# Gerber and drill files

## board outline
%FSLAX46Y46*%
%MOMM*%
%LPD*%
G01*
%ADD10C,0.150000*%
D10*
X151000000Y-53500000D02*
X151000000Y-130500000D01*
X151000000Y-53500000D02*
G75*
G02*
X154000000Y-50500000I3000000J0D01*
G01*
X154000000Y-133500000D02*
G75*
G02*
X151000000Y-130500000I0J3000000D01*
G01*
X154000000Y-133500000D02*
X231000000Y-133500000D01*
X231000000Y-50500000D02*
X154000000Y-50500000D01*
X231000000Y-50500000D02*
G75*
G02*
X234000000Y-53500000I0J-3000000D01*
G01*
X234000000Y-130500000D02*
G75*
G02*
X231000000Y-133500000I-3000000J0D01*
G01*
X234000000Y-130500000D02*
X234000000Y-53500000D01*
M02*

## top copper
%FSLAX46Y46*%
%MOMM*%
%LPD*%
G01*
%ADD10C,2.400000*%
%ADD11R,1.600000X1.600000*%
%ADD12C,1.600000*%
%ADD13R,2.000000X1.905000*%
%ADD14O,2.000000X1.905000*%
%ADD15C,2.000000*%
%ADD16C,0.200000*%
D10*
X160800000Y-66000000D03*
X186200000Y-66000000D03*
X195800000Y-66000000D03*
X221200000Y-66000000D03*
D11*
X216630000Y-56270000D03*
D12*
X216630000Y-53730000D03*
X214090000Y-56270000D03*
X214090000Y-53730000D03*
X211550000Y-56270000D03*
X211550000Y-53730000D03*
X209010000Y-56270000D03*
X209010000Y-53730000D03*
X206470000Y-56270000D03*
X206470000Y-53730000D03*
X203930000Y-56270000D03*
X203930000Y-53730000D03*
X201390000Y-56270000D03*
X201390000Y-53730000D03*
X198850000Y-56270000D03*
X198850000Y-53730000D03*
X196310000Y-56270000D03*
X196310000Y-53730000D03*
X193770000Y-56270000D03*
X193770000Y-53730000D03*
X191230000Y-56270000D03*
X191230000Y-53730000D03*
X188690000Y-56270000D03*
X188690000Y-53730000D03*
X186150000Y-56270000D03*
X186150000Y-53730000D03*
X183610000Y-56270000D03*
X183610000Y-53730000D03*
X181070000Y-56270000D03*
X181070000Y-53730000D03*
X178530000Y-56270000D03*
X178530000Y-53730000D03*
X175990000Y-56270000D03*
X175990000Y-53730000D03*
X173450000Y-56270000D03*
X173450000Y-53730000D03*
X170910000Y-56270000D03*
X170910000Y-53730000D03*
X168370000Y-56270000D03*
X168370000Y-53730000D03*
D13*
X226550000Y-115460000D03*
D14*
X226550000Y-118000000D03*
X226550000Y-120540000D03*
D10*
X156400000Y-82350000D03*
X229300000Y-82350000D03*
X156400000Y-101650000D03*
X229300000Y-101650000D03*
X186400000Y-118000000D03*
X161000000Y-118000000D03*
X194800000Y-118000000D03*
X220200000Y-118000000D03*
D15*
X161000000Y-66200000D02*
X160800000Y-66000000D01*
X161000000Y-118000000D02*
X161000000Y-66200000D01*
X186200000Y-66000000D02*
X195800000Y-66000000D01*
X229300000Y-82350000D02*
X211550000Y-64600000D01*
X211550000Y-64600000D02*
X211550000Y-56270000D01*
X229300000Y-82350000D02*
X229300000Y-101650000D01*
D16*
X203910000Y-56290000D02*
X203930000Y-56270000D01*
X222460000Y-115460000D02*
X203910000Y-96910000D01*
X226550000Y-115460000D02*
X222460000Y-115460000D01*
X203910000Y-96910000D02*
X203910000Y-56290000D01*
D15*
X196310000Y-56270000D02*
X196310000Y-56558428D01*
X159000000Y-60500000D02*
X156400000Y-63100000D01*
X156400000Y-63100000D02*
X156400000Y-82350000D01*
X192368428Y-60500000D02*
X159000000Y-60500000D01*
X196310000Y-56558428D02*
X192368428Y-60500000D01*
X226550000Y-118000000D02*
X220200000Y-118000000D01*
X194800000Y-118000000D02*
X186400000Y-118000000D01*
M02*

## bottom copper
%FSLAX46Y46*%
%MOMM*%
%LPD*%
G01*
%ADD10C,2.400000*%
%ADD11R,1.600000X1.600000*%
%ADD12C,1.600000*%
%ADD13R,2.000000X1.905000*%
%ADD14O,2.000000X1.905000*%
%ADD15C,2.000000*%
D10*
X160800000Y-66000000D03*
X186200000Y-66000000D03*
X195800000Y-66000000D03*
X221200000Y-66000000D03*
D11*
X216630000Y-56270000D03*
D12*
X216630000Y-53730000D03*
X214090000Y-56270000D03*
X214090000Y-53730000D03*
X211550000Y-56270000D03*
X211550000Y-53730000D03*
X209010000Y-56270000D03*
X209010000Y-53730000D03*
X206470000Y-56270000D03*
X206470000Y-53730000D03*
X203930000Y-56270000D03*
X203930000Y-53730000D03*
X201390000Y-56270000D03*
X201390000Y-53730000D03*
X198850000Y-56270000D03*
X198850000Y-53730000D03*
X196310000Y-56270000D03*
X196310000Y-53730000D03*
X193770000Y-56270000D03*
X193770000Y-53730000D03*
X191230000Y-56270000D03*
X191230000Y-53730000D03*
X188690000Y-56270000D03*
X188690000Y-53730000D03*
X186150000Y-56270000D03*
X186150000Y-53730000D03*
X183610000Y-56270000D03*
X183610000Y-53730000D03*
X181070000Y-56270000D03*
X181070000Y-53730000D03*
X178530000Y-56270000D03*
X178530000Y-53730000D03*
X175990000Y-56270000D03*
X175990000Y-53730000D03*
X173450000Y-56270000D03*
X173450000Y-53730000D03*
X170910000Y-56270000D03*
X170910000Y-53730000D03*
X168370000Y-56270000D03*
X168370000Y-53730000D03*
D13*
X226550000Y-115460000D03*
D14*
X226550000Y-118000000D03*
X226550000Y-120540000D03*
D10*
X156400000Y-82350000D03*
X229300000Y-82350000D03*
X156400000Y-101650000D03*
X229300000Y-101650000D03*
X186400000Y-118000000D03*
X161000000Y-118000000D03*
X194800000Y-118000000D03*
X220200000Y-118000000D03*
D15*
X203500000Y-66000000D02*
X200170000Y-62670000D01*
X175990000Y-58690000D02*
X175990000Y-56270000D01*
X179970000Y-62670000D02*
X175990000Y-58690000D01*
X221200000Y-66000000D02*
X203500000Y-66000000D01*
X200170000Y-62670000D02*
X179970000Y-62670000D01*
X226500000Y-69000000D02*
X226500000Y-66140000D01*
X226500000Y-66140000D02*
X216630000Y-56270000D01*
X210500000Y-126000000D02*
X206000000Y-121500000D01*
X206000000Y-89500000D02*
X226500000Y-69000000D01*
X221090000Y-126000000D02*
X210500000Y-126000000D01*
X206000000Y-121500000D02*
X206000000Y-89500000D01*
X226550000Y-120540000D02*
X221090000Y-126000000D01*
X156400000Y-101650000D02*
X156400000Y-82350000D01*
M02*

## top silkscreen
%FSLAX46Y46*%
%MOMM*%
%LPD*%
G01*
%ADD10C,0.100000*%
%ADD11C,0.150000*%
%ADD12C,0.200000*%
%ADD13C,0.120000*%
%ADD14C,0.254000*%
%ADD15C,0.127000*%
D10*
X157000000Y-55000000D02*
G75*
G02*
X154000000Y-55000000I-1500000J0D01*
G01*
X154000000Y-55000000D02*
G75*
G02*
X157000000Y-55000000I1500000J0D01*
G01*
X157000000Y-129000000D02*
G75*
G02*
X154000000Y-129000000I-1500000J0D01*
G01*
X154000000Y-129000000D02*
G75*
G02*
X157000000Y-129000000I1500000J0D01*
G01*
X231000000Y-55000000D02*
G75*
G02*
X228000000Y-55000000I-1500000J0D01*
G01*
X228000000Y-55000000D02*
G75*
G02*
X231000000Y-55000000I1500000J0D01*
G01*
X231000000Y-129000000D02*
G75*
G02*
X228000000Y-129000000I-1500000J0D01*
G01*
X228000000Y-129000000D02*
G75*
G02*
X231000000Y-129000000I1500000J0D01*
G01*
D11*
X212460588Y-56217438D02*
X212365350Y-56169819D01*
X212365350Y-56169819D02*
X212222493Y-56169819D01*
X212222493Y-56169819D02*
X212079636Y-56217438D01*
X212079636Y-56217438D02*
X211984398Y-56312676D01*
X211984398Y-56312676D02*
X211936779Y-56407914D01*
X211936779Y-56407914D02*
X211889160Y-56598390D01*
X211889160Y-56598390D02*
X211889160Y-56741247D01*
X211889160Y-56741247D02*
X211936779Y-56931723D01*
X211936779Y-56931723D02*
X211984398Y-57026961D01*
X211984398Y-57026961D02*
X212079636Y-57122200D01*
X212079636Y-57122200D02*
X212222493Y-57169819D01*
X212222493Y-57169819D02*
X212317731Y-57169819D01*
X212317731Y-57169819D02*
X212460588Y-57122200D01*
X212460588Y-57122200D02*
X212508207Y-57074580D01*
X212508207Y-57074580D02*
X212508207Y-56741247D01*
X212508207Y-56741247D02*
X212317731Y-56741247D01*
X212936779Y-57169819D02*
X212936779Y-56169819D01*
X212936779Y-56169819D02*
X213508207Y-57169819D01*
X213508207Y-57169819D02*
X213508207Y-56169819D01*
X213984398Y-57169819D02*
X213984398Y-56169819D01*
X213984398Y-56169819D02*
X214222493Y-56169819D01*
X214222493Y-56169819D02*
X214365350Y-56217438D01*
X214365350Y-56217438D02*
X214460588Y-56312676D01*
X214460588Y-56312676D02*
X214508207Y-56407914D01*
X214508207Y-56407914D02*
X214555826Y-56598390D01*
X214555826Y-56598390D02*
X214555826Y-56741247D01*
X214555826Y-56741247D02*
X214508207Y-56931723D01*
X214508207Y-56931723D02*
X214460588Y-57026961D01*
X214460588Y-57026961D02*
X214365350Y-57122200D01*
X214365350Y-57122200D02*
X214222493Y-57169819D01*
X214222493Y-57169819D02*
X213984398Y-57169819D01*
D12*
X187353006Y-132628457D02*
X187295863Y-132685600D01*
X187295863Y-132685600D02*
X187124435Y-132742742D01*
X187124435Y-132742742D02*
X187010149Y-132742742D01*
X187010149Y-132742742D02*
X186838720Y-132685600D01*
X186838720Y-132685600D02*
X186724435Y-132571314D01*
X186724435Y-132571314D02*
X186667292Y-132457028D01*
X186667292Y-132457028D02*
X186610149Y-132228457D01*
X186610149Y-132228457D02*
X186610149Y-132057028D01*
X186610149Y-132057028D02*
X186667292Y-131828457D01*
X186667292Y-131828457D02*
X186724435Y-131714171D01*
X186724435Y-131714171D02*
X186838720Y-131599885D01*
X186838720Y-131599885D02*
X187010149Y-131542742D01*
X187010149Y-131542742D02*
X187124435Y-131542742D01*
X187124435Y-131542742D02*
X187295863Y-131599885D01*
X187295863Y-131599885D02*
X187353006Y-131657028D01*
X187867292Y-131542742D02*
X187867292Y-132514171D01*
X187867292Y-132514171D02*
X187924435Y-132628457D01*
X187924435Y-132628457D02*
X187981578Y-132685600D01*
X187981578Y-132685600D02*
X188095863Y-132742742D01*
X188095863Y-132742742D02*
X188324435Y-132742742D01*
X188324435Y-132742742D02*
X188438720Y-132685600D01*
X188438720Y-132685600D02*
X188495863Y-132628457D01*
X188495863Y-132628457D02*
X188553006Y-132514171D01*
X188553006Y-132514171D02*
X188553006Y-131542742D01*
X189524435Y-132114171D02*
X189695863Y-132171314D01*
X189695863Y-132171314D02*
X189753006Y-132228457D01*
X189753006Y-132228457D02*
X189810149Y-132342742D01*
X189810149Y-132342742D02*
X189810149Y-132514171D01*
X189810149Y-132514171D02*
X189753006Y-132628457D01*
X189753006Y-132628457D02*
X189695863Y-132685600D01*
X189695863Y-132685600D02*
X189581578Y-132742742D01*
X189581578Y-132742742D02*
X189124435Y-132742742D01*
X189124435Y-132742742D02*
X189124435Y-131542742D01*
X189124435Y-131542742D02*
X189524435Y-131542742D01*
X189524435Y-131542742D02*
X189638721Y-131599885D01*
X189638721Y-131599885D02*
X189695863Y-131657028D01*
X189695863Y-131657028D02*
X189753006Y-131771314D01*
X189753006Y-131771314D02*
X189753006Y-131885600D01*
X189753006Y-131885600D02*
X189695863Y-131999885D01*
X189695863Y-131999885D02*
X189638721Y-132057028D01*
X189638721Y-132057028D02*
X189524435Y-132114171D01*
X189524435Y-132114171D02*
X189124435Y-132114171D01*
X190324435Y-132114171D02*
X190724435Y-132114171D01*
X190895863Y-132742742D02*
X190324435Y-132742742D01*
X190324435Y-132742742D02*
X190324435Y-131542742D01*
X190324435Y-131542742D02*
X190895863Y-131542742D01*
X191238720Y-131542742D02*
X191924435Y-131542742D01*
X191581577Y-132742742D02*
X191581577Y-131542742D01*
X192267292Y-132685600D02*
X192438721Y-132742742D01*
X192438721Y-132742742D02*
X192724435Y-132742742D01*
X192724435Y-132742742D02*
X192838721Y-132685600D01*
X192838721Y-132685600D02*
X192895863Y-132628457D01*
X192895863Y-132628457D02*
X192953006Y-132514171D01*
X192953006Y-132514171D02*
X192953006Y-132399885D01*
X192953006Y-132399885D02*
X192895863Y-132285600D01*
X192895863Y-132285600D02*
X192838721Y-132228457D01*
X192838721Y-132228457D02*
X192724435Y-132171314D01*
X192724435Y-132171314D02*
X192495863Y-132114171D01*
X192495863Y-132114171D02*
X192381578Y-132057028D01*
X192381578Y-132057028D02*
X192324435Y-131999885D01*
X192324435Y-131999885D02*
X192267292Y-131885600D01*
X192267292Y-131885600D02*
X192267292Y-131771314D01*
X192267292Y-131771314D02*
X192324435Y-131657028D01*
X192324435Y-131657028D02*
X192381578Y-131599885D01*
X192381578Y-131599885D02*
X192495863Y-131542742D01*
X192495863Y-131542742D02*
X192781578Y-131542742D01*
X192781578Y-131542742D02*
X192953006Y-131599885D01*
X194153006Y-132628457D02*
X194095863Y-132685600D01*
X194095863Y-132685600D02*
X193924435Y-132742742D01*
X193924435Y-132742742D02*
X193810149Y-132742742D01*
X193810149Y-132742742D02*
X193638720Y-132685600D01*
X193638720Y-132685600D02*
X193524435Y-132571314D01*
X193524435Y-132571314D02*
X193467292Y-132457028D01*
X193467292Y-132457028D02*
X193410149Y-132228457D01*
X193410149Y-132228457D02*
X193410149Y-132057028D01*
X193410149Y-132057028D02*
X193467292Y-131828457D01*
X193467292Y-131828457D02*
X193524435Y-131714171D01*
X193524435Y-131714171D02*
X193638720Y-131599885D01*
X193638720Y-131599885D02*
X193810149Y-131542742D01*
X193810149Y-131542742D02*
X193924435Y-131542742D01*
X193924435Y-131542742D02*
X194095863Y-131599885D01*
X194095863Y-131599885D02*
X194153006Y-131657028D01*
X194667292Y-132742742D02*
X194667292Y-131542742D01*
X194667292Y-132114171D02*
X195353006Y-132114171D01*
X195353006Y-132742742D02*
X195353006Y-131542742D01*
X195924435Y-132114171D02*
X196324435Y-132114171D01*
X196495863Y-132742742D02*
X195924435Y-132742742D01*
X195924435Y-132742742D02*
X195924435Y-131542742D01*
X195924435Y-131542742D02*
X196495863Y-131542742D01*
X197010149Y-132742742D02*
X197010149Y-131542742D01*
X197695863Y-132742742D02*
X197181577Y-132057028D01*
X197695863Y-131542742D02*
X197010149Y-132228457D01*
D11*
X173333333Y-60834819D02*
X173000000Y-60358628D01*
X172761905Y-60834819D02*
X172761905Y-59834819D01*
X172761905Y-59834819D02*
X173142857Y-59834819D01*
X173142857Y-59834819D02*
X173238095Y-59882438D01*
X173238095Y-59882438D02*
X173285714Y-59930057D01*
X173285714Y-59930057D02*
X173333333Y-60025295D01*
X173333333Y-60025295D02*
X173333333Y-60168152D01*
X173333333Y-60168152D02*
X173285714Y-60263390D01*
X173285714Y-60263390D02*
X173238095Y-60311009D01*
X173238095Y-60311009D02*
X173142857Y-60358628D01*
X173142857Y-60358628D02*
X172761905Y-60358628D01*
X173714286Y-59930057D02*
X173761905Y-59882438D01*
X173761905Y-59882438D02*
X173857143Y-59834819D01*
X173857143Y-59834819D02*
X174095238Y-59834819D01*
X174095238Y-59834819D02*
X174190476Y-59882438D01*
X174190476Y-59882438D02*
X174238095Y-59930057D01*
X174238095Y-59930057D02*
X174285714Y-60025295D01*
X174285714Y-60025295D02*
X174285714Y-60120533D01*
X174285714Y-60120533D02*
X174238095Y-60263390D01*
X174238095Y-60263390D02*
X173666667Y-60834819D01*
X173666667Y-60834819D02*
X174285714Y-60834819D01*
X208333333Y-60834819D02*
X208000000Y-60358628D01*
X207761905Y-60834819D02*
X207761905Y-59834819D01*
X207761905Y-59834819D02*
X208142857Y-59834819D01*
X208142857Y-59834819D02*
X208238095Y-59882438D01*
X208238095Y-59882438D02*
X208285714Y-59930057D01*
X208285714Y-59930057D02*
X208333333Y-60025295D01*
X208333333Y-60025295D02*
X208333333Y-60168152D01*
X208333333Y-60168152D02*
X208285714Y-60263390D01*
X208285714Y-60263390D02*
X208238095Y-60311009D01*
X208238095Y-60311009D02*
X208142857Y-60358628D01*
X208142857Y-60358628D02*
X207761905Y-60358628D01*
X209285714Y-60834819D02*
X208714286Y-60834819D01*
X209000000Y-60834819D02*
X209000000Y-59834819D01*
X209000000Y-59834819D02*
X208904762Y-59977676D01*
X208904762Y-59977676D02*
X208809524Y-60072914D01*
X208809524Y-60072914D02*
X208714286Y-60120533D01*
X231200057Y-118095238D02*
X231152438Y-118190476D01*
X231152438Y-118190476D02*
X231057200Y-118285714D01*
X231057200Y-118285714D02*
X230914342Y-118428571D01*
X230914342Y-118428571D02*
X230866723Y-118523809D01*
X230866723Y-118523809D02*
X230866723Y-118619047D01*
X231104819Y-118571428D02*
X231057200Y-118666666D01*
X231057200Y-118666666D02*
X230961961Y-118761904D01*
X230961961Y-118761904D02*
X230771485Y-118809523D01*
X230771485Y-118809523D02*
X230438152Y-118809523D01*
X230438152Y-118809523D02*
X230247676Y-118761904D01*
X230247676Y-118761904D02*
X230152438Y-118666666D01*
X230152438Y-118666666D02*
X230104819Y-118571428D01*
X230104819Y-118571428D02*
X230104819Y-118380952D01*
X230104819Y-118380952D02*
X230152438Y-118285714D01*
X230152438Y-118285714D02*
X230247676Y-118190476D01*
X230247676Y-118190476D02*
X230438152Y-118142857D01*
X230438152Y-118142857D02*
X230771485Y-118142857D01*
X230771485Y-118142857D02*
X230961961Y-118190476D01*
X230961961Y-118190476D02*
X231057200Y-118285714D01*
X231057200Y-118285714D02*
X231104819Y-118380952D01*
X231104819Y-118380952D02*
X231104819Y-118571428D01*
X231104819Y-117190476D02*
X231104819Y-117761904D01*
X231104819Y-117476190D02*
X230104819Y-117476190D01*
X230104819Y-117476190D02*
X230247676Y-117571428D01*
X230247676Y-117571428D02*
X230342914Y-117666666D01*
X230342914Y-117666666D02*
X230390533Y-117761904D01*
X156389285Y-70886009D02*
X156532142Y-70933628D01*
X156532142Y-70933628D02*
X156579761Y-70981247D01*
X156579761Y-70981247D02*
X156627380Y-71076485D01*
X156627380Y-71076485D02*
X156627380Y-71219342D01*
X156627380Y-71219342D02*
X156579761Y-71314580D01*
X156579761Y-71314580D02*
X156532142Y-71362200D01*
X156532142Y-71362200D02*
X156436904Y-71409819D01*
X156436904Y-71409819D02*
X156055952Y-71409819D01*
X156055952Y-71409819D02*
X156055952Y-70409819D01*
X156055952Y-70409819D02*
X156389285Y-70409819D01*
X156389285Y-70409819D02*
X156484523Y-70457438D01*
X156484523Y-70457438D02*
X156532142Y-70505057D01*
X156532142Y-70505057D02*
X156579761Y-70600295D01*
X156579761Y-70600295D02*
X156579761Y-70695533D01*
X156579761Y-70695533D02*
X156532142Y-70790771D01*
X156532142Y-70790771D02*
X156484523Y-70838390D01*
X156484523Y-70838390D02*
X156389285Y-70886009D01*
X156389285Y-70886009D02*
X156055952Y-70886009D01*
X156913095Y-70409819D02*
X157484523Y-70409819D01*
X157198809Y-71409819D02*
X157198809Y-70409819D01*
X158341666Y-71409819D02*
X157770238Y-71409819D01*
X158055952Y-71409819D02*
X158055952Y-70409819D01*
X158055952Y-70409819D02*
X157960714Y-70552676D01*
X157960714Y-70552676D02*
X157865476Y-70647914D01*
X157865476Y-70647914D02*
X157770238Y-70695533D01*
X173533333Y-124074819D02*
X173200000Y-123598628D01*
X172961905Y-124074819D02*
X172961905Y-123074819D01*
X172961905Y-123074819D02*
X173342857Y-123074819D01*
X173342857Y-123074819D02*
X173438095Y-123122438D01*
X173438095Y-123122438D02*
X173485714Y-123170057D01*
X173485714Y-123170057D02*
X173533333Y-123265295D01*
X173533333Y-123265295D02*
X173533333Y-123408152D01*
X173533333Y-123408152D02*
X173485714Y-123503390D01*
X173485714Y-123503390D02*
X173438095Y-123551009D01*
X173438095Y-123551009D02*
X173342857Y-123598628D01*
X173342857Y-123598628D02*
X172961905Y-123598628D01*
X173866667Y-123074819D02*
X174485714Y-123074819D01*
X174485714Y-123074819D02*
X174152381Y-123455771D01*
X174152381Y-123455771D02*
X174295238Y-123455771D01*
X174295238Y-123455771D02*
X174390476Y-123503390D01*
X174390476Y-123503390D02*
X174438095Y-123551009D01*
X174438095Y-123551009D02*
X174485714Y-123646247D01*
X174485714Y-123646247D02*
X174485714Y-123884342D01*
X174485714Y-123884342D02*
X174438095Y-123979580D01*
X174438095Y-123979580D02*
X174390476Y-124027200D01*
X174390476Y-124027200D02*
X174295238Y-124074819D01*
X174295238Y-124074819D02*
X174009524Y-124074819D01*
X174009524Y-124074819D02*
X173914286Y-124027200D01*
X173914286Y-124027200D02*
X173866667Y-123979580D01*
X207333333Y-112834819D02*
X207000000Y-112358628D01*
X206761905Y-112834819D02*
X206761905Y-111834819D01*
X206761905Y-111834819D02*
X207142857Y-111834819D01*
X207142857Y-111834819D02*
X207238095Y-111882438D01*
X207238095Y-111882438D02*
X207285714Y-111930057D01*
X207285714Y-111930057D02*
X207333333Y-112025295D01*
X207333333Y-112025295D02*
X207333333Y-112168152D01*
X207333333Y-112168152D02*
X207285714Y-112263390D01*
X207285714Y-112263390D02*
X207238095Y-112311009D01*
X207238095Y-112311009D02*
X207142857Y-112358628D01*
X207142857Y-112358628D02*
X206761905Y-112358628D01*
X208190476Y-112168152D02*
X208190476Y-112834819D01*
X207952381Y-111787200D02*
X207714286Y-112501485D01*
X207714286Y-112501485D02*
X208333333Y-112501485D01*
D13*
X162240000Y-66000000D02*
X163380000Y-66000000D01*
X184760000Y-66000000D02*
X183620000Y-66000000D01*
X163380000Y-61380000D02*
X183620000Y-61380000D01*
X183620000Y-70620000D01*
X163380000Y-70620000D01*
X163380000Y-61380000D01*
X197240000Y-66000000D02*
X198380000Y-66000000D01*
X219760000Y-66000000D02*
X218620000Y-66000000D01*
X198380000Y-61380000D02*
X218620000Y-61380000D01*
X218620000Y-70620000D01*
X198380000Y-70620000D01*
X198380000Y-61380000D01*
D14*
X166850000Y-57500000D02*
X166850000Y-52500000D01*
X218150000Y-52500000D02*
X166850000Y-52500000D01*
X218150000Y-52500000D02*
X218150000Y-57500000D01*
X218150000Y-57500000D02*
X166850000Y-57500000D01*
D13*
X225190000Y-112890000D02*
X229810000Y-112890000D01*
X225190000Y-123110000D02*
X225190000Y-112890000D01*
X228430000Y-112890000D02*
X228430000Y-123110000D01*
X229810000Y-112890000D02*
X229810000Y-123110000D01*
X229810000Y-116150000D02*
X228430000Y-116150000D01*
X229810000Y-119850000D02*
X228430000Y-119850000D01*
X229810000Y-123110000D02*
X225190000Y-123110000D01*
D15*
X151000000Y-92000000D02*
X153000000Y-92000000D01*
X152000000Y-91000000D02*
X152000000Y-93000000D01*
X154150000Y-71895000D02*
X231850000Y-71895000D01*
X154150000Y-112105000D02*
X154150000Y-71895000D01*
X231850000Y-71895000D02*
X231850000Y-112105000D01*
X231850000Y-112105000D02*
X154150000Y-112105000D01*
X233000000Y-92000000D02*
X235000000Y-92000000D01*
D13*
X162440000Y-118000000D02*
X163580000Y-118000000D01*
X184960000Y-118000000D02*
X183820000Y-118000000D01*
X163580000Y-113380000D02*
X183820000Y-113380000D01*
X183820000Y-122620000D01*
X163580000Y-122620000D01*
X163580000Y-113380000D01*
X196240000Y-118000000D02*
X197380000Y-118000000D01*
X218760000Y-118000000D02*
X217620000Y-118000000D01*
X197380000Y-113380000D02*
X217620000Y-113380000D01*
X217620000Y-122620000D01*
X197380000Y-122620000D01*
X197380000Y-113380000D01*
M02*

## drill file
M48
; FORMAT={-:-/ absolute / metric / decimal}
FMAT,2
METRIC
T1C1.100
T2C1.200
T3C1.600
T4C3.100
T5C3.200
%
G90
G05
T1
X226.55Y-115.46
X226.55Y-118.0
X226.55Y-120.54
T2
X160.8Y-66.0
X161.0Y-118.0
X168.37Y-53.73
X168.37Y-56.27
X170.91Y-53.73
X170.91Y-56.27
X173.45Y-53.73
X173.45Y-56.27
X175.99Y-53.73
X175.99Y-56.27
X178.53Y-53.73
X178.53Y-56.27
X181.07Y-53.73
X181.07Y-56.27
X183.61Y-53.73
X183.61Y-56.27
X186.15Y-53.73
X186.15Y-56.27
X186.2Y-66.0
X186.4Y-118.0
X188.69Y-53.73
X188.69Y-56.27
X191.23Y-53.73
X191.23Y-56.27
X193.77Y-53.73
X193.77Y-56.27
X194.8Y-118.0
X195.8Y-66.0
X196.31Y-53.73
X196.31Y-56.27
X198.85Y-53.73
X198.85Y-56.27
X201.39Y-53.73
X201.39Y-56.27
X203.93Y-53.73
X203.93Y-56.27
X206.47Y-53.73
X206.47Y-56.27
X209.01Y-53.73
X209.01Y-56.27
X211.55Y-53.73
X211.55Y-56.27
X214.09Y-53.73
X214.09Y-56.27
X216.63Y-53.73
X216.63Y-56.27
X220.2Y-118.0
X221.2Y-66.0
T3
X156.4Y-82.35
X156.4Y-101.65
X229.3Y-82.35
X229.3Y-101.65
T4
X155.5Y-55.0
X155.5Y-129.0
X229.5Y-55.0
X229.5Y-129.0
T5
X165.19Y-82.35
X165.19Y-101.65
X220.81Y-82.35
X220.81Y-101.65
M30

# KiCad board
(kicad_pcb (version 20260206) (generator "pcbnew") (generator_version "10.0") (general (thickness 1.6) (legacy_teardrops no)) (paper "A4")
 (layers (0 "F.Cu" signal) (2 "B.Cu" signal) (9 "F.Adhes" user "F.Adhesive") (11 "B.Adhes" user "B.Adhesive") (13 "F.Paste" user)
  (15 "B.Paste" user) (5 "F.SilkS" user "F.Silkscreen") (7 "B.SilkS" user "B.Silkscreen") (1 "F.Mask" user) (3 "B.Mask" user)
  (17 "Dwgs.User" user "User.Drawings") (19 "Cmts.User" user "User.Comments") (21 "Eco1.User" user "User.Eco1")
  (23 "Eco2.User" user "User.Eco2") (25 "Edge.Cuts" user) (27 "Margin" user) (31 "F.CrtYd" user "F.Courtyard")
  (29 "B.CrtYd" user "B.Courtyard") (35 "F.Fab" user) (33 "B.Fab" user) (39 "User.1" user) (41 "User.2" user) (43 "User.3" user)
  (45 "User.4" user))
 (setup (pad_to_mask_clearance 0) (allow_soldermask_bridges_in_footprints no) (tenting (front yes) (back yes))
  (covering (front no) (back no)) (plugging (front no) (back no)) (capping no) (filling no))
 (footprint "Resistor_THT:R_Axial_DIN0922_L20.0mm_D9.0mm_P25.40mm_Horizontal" (layer "F.Cu") (at 160.8 66)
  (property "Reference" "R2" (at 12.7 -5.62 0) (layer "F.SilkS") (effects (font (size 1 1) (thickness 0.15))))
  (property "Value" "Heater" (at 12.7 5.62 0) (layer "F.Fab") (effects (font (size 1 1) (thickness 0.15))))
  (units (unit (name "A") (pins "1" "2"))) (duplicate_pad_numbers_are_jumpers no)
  (fp_line (start 1.44 0) (end 2.58 0) (stroke (width 0.12) (type solid)) (layer "F.SilkS"))
  (fp_line (start 23.96 0) (end 22.82 0) (stroke (width 0.12) (type solid)) (layer "F.SilkS"))
  (fp_rect (start 2.58 -4.62) (end 22.82 4.62) (stroke (width 0.12) (type solid)) (fill no) (layer "F.SilkS"))
  (pad "1" thru_hole circle (at 0 0) (size 2.4 2.4) (drill 1.2) (layers "*.Cu" "*.Mask") (remove_unused_layers no) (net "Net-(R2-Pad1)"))
  (pad "2" thru_hole circle (at 25.4 0) (size 2.4 2.4) (drill 1.2) (layers "*.Cu" "*.Mask") (remove_unused_layers no) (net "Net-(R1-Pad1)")))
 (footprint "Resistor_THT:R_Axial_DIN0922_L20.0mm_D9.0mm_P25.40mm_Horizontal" (layer "F.Cu") (at 195.8 66)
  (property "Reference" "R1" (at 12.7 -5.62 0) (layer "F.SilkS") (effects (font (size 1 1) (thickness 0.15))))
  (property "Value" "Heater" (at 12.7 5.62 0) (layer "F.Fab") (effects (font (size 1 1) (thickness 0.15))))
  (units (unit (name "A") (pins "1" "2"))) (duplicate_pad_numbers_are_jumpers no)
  (fp_line (start 1.44 0) (end 2.58 0) (stroke (width 0.12) (type solid)) (layer "F.SilkS"))
  (fp_line (start 23.96 0) (end 22.82 0) (stroke (width 0.12) (type solid)) (layer "F.SilkS"))
  (fp_rect (start 2.58 -4.62) (end 22.82 4.62) (stroke (width 0.12) (type solid)) (fill no) (layer "F.SilkS"))
  (pad "1" thru_hole circle (at 0 0) (size 2.4 2.4) (drill 1.2) (layers "*.Cu" "*.Mask") (remove_unused_layers no) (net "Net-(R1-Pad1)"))
  (pad "2" thru_hole circle (at 25.4 0) (size 2.4 2.4) (drill 1.2) (layers "*.Cu" "*.Mask") (remove_unused_layers no) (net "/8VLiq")))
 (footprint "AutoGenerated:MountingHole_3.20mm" (layer "F.Cu") (at 155.5 129)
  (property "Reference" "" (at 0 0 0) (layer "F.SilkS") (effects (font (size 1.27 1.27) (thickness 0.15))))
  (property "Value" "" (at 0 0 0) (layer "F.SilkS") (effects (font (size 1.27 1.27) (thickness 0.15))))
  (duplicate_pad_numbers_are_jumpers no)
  (pad "" np_thru_hole circle (at 0 0) (size 3.1 3.1) (drill 3.1) (layers "*.Cu" "*.Mask")))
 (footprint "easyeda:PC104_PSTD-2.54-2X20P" (layer "F.Cu") (at 216.63 53.73 -90)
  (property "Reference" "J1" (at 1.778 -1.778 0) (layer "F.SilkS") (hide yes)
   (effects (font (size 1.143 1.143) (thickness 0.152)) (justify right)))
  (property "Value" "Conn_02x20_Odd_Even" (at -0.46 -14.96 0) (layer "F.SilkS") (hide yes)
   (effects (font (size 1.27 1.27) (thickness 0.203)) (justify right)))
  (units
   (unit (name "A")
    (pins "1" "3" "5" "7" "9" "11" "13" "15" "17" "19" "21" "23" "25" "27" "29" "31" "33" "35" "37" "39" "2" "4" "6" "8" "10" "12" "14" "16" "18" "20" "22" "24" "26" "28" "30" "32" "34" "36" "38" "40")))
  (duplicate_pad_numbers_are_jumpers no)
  (fp_line (start 3.77 49.78) (end -1.23 49.78) (stroke (width 0.254) (type solid)) (layer "F.SilkS"))
  (fp_line (start -1.23 -1.52) (end -1.23 49.78) (stroke (width 0.254) (type solid)) (layer "F.SilkS"))
  (fp_line (start -1.23 -1.52) (end 3.77 -1.52) (stroke (width 0.254) (type solid)) (layer "F.SilkS"))
  (fp_line (start 3.77 -1.52) (end 3.77 49.78) (stroke (width 0.254) (type solid)) (layer "F.SilkS"))
  (pad "1" thru_hole rect (at 2.54 0 180) (size 1.6 1.6) (drill 1.2) (layers "*.Cu" "*.Paste" "*.Mask") (remove_unused_layers no)
   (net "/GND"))
  (pad "2" thru_hole circle (at 0 0 180) (size 1.6 1.6) (drill 1.2) (layers "*.Cu" "*.Paste" "*.Mask") (remove_unused_layers no)
   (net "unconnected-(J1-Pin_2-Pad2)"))
  (pad "3" thru_hole circle (at 2.54 2.54 180) (size 1.6 1.6) (drill 1.2) (layers "*.Cu" "*.Paste" "*.Mask") (remove_unused_layers no)
   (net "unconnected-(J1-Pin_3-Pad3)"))
  (pad "4" thru_hole circle (at 0 2.54 180) (size 1.6 1.6) (drill 1.2) (layers "*.Cu" "*.Paste" "*.Mask") (remove_unused_layers no)
   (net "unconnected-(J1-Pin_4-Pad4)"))
  (pad "5" thru_hole circle (at 2.54 5.08 180) (size 1.6 1.6) (drill 1.2) (layers "*.Cu" "*.Paste" "*.Mask") (remove_unused_layers no)
   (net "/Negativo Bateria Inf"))
  (pad "6" thru_hole circle (at 0 5.08 180) (size 1.6 1.6) (drill 1.2) (layers "*.Cu" "*.Paste" "*.Mask") (remove_unused_layers no)
   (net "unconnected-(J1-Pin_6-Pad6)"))
  (pad "7" thru_hole circle (at 2.54 7.62 180) (size 1.6 1.6) (drill 1.2) (layers "*.Cu" "*.Paste" "*.Mask") (remove_unused_layers no)
   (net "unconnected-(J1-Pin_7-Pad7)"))
  (pad "8" thru_hole circle (at 0 7.62 180) (size 1.6 1.6) (drill 1.2) (layers "*.Cu" "*.Paste" "*.Mask") (remove_unused_layers no)
   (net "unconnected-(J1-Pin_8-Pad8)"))
  (pad "9" thru_hole circle (at 2.54 10.16 180) (size 1.6 1.6) (drill 1.2) (layers "*.Cu" "*.Paste" "*.Mask") (remove_unused_layers no)
   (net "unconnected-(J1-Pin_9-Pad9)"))
  (pad "10" thru_hole circle (at 0 10.16 180) (size 1.6 1.6) (drill 1.2) (layers "*.Cu" "*.Paste" "*.Mask") (remove_unused_layers no)
   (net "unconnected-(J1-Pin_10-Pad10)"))
  (pad "11" thru_hole circle (at 2.54 12.7 180) (size 1.6 1.6) (drill 1.2) (layers "*.Cu" "*.Paste" "*.Mask") (remove_unused_layers no)
   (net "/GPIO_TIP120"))
  (pad "12" thru_hole circle (at 0 12.7 180) (size 1.6 1.6) (drill 1.2) (layers "*.Cu" "*.Paste" "*.Mask") (remove_unused_layers no)
   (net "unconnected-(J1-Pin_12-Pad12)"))
  (pad "13" thru_hole circle (at 2.54 15.24 180) (size 1.6 1.6) (drill 1.2) (layers "*.Cu" "*.Paste" "*.Mask") (remove_unused_layers no)
   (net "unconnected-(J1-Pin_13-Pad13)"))
  (pad "14" thru_hole circle (at 0 15.24 180) (size 1.6 1.6) (drill 1.2) (layers "*.Cu" "*.Paste" "*.Mask") (remove_unused_layers no)
   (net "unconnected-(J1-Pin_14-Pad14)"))
  (pad "15" thru_hole circle (at 2.54 17.78 180) (size 1.6 1.6) (drill 1.2) (layers "*.Cu" "*.Paste" "*.Mask") (remove_unused_layers no)
   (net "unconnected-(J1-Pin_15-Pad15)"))
  (pad "16" thru_hole circle (at 0 17.78 180) (size 1.6 1.6) (drill 1.2) (layers "*.Cu" "*.Paste" "*.Mask") (remove_unused_layers no)
   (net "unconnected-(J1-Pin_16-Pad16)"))
  (pad "17" thru_hole circle (at 2.54 20.32 180) (size 1.6 1.6) (drill 1.2) (layers "*.Cu" "*.Paste" "*.Mask") (remove_unused_layers no)
   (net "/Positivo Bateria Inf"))
  (pad "18" thru_hole circle (at 0 20.32 180) (size 1.6 1.6) (drill 1.2) (layers "*.Cu" "*.Paste" "*.Mask") (remove_unused_layers no)
   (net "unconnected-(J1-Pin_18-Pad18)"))
  (pad "19" thru_hole circle (at 2.54 22.86 180) (size 1.6 1.6) (drill 1.2) (layers "*.Cu" "*.Paste" "*.Mask") (remove_unused_layers no)
   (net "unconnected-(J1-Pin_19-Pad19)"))
  (pad "20" thru_hole circle (at 0 22.86 180) (size 1.6 1.6) (drill 1.2) (layers "*.Cu" "*.Paste" "*.Mask") (remove_unused_layers no)
   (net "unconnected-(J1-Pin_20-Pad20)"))
  (pad "21" thru_hole circle (at 2.54 25.4 180) (size 1.6 1.6) (drill 1.2) (layers "*.Cu" "*.Paste" "*.Mask") (remove_unused_layers no)
   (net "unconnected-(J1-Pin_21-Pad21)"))
  (pad "22" thru_hole circle (at 0 25.4 180) (size 1.6 1.6) (drill 1.2) (layers "*.Cu" "*.Paste" "*.Mask") (remove_unused_layers no)
   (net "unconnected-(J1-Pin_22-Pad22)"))
  (pad "23" thru_hole circle (at 2.54 27.94 180) (size 1.6 1.6) (drill 1.2) (layers "*.Cu" "*.Paste" "*.Mask") (remove_unused_layers no)
   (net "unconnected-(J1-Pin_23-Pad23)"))
  (pad "24" thru_hole circle (at 0 27.94 180) (size 1.6 1.6) (drill 1.2) (layers "*.Cu" "*.Paste" "*.Mask") (remove_unused_layers no)
   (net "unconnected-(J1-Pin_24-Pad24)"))
  (pad "25" thru_hole circle (at 2.54 30.48 180) (size 1.6 1.6) (drill 1.2) (layers "*.Cu" "*.Paste" "*.Mask") (remove_unused_layers no)
   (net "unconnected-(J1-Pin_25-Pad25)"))
  (pad "26" thru_hole circle (at 0 30.48 180) (size 1.6 1.6) (drill 1.2) (layers "*.Cu" "*.Paste" "*.Mask") (remove_unused_layers no)
   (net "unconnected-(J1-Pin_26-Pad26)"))
  (pad "27" thru_hole circle (at 2.54 33.02 180) (size 1.6 1.6) (drill 1.2) (layers "*.Cu" "*.Paste" "*.Mask") (remove_unused_layers no)
   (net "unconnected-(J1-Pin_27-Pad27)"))
  (pad "28" thru_hole circle (at 0 33.02 180) (size 1.6 1.6) (drill 1.2) (layers "*.Cu" "*.Paste" "*.Mask") (remove_unused_layers no)
   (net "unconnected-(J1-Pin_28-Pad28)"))
  (pad "29" thru_hole circle (at 2.54 35.56 180) (size 1.6 1.6) (drill 1.2) (layers "*.Cu" "*.Paste" "*.Mask") (remove_unused_layers no)
   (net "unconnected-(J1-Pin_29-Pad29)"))
  (pad "30" thru_hole circle (at 0 35.56 180) (size 1.6 1.6) (drill 1.2) (layers "*.Cu" "*.Paste" "*.Mask") (remove_unused_layers no)
   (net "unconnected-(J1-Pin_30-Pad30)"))
  (pad "31" thru_hole circle (at 2.54 38.1 180) (size 1.6 1.6) (drill 1.2) (layers "*.Cu" "*.Paste" "*.Mask") (remove_unused_layers no)
   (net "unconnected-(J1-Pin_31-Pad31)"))
  (pad "32" thru_hole circle (at 0 38.1 180) (size 1.6 1.6) (drill 1.2) (layers "*.Cu" "*.Paste" "*.Mask") (remove_unused_layers no)
   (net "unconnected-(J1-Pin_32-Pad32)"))
  (pad "33" thru_hole circle (at 2.54 40.64 180) (size 1.6 1.6) (drill 1.2) (layers "*.Cu" "*.Paste" "*.Mask") (remove_unused_layers no)
   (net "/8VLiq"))
  (pad "34" thru_hole circle (at 0 40.64 180) (size 1.6 1.6) (drill 1.2) (layers "*.Cu" "*.Paste" "*.Mask") (remove_unused_layers no)
   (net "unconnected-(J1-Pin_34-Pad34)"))
  (pad "35" thru_hole circle (at 2.54 43.18 180) (size 1.6 1.6) (drill 1.2) (layers "*.Cu" "*.Paste" "*.Mask") (remove_unused_layers no)
   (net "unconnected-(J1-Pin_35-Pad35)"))
  (pad "36" thru_hole circle (at 0 43.18 180) (size 1.6 1.6) (drill 1.2) (layers "*.Cu" "*.Paste" "*.Mask") (remove_unused_layers no)
   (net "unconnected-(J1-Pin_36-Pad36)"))
  (pad "37" thru_hole circle (at 2.54 45.72 180) (size 1.6 1.6) (drill 1.2) (layers "*.Cu" "*.Paste" "*.Mask") (remove_unused_layers no)
   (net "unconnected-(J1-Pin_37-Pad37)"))
  (pad "38" thru_hole circle (at 0 45.72 180) (size 1.6 1.6) (drill 1.2) (layers "*.Cu" "*.Paste" "*.Mask") (remove_unused_layers no)
   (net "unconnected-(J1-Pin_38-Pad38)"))
  (pad "39" thru_hole circle (at 2.54 48.26 180) (size 1.6 1.6) (drill 1.2) (layers "*.Cu" "*.Paste" "*.Mask") (remove_unused_layers no)
   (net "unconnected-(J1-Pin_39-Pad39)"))
  (pad "40" thru_hole circle (at 0 48.26 180) (size 1.6 1.6) (drill 1.2) (layers "*.Cu" "*.Paste" "*.Mask") (remove_unused_layers no)
   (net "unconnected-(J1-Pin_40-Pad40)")))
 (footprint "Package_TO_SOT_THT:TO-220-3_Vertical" (layer "F.Cu") (at 226.55 115.46 -90)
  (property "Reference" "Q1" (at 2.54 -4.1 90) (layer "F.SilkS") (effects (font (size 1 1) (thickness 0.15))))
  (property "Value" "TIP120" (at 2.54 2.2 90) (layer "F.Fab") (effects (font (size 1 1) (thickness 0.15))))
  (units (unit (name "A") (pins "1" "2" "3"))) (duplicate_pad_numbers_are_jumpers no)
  (fp_line (start -2.57 1.36) (end -2.57 -3.26) (stroke (width 0.12) (type solid)) (layer "F.SilkS"))
  (fp_line (start 7.65 1.36) (end -2.57 1.36) (stroke (width 0.12) (type solid)) (layer "F.SilkS"))
  (fp_line (start -2.57 -1.88) (end 7.65 -1.88) (stroke (width 0.12) (type solid)) (layer "F.SilkS"))
  (fp_line (start -2.57 -3.26) (end 7.65 -3.26) (stroke (width 0.12) (type solid)) (layer "F.SilkS"))
  (fp_line (start 0.69 -3.26) (end 0.69 -1.88) (stroke (width 0.12) (type solid)) (layer "F.SilkS"))
  (fp_line (start 4.39 -3.26) (end 4.39 -1.88) (stroke (width 0.12) (type solid)) (layer "F.SilkS"))
  (fp_line (start 7.65 -3.26) (end 7.65 1.36) (stroke (width 0.12) (type solid)) (layer "F.SilkS"))
  (pad "1" thru_hole rect (at 0 0 270) (size 1.905 2) (drill 1.1) (layers "*.Cu" "*.Mask") (remove_unused_layers no) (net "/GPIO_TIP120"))
  (pad "2" thru_hole oval (at 2.54 0 270) (size 1.905 2) (drill 1.1) (layers "*.Cu" "*.Mask") (remove_unused_layers no) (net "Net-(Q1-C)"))
  (pad "3" thru_hole oval (at 5.08 0 270) (size 1.905 2) (drill 1.1) (layers "*.Cu" "*.Mask") (remove_unused_layers no) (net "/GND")))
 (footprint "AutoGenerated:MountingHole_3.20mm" (layer "F.Cu") (at 229.5 55)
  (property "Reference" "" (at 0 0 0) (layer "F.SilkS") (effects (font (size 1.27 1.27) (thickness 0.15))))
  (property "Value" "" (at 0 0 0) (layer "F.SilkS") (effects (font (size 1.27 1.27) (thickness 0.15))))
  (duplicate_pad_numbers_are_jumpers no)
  (pad "" np_thru_hole circle (at 0 0) (size 3.1 3.1) (drill 3.1) (layers "*.Cu" "*.Mask")))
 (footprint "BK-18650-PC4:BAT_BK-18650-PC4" (layer "F.Cu") (at 193 92)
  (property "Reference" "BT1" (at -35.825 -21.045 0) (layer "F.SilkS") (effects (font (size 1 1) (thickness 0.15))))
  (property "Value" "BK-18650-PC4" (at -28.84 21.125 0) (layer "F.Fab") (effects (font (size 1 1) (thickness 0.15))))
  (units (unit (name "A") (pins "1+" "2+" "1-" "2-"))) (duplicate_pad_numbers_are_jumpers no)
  (fp_line (start -42 0) (end -40 0) (stroke (width 0.127) (type solid)) (layer "F.SilkS"))
  (fp_line (start -41 -1) (end -41 1) (stroke (width 0.127) (type solid)) (layer "F.SilkS"))
  (fp_line (start -38.85 -20.105) (end 38.85 -20.105) (stroke (width 0.127) (type solid)) (layer "F.SilkS"))
  (fp_line (start -38.85 20.105) (end -38.85 -20.105) (stroke (width 0.127) (type solid)) (layer "F.SilkS"))
  (fp_line (start 38.85 -20.105) (end 38.85 20.105) (stroke (width 0.127) (type solid)) (layer "F.SilkS"))
  (fp_line (start 38.85 20.105) (end -38.85 20.105) (stroke (width 0.127) (type solid)) (layer "F.SilkS"))
  (fp_line (start 40 0) (end 42 0) (stroke (width 0.127) (type solid)) (layer "F.SilkS"))
  (pad "" np_thru_hole circle (at -27.81 -9.65) (size 3.2 3.2) (drill 3.2) (layers "*.Cu" "*.Mask"))
  (pad "" np_thru_hole circle (at -27.81 9.65) (size 3.2 3.2) (drill 3.2) (layers "*.Cu" "*.Mask"))
  (pad "" np_thru_hole circle (at 27.81 -9.65) (size 3.2 3.2) (drill 3.2) (layers "*.Cu" "*.Mask"))
  (pad "" np_thru_hole circle (at 27.81 9.65) (size 3.2 3.2) (drill 3.2) (layers "*.Cu" "*.Mask"))
  (pad "1+" thru_hole circle (at -36.6 -9.65) (size 2.4 2.4) (drill 1.6) (layers "*.Cu" "*.Mask") (remove_unused_layers no)
   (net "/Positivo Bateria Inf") (solder_mask_margin 0.102))
  (pad "1-" thru_hole circle (at 36.3 -9.65) (size 2.4 2.4) (drill 1.6) (layers "*.Cu" "*.Mask") (remove_unused_layers no)
   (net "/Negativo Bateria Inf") (solder_mask_margin 0.102))
  (pad "2+" thru_hole circle (at -36.6 9.65) (size 2.4 2.4) (drill 1.6) (layers "*.Cu" "*.Mask") (remove_unused_layers no)
   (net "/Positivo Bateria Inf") (solder_mask_margin 0.102))
  (pad "2-" thru_hole circle (at 36.3 9.65) (size 2.4 2.4) (drill 1.6) (layers "*.Cu" "*.Mask") (remove_unused_layers no)
   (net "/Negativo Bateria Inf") (solder_mask_margin 0.102)))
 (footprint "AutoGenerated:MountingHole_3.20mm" (layer "F.Cu") (at 229.5 129)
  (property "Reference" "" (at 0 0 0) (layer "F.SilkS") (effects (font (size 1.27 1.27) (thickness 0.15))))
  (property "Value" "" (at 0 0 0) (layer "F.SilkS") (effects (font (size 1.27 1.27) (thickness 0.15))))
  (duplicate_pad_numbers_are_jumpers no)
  (pad "" np_thru_hole circle (at 0 0) (size 3.1 3.1) (drill 3.1) (layers "*.Cu" "*.Mask")))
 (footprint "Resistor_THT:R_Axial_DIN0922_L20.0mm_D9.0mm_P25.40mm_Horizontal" (layer "F.Cu") (at 186.4 118 180)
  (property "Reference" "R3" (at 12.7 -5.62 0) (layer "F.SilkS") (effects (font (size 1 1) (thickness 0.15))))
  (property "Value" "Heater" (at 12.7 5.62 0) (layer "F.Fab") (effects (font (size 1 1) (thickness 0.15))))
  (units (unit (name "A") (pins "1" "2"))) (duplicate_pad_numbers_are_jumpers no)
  (fp_line (start 23.96 0) (end 22.82 0) (stroke (width 0.12) (type solid)) (layer "F.SilkS"))
  (fp_line (start 1.44 0) (end 2.58 0) (stroke (width 0.12) (type solid)) (layer "F.SilkS"))
  (fp_rect (start 2.58 -4.62) (end 22.82 4.62) (stroke (width 0.12) (type solid)) (fill no) (layer "F.SilkS"))
  (pad "1" thru_hole circle (at 0 0 180) (size 2.4 2.4) (drill 1.2) (layers "*.Cu" "*.Mask") (remove_unused_layers no) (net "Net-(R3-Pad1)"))
  (pad "2" thru_hole circle (at 25.4 0 180) (size 2.4 2.4) (drill 1.2) (layers "*.Cu" "*.Mask") (remove_unused_layers no)
   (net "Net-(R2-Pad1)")))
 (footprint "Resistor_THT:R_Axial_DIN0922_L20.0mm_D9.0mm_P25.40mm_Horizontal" (layer "F.Cu") (at 194.8 118)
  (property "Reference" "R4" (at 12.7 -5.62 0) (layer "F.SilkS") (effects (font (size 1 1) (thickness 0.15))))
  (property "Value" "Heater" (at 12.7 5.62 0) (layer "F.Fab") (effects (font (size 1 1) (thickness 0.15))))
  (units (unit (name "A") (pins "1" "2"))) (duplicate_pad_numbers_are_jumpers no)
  (fp_line (start 1.44 0) (end 2.58 0) (stroke (width 0.12) (type solid)) (layer "F.SilkS"))
  (fp_line (start 23.96 0) (end 22.82 0) (stroke (width 0.12) (type solid)) (layer "F.SilkS"))
  (fp_rect (start 2.58 -4.62) (end 22.82 4.62) (stroke (width 0.12) (type solid)) (fill no) (layer "F.SilkS"))
  (pad "1" thru_hole circle (at 0 0) (size 2.4 2.4) (drill 1.2) (layers "*.Cu" "*.Mask") (remove_unused_layers no) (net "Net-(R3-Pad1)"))
  (pad "2" thru_hole circle (at 25.4 0) (size 2.4 2.4) (drill 1.2) (layers "*.Cu" "*.Mask") (remove_unused_layers no) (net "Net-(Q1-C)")))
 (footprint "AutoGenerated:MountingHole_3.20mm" (layer "F.Cu") (at 155.5 55)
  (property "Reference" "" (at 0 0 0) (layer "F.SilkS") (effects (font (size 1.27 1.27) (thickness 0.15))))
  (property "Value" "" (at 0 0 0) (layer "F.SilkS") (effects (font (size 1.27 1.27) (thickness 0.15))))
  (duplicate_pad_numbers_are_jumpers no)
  (pad "" np_thru_hole circle (at 0 0) (size 3.1 3.1) (drill 3.1) (layers "*.Cu" "*.Mask")))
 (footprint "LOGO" (layer "B.Cu") (at 221.64 131.81 180)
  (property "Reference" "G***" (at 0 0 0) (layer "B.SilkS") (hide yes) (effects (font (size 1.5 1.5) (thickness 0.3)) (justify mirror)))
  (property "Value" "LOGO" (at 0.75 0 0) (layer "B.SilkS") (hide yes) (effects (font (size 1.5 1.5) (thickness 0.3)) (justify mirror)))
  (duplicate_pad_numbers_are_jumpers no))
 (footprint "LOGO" (layer "B.Cu") (at 162.08 131.86 180)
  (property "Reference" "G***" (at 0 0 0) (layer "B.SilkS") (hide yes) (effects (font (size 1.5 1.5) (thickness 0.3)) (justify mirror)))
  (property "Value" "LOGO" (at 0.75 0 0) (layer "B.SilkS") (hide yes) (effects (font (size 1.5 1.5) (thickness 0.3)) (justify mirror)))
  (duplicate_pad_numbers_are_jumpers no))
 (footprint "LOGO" (layer "B.Cu") (at 175 130 180)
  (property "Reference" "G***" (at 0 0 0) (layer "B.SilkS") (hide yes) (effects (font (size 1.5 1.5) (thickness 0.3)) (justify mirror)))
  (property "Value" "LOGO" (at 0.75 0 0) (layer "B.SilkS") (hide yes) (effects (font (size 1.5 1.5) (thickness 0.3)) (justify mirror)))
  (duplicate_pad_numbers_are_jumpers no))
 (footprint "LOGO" (layer "B.Cu") (at 210.27 129.9 90)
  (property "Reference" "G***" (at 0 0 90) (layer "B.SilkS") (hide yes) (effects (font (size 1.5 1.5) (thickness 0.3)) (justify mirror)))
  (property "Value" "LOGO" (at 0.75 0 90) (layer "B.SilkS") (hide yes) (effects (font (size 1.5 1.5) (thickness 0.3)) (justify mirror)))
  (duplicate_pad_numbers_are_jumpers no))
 (gr_circle (center 155.5 55) (end 157 55) (stroke (width 0.1) (type solid)) (fill no) (layer "F.SilkS"))
 (gr_circle (center 155.5 129) (end 157 129) (stroke (width 0.1) (type solid)) (fill no) (layer "F.SilkS"))
 (gr_circle (center 229.5 55) (end 231 55) (stroke (width 0.1) (type solid)) (fill no) (layer "F.SilkS"))
 (gr_circle (center 229.5 129) (end 231 129) (stroke (width 0.1) (type default)) (fill no) (layer "F.SilkS"))
 (gr_line (start 151 53.5) (end 151 130.5) (stroke (width 0.15) (type solid)) (layer "Edge.Cuts"))
 (gr_arc (start 151 53.5) (mid 151.87868 51.37868) (end 154 50.5) (stroke (width 0.15) (type solid)) (layer "Edge.Cuts"))
 (gr_arc (start 154 133.5) (mid 151.87868 132.62132) (end 151 130.5) (stroke (width 0.15) (type solid)) (layer "Edge.Cuts"))
 (gr_line (start 154 133.5) (end 231 133.5) (stroke (width 0.15) (type solid)) (layer "Edge.Cuts"))
 (gr_line (start 231 50.5) (end 154 50.5) (stroke (width 0.15) (type solid)) (layer "Edge.Cuts"))
 (gr_arc (start 231 50.5) (mid 233.12132 51.37868) (end 234 53.5) (stroke (width 0.15) (type solid)) (layer "Edge.Cuts"))
 (gr_arc (start 234 130.5) (mid 233.12132 132.62132) (end 231 133.5) (stroke (width 0.15) (type solid)) (layer "Edge.Cuts"))
 (gr_line (start 234 130.5) (end 234 53.5) (stroke (width 0.15) (type solid)) (layer "Edge.Cuts"))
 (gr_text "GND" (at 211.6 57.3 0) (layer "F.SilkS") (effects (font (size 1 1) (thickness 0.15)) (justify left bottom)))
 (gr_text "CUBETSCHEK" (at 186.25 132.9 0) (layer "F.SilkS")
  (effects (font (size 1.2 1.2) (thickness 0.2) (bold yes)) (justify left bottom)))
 (segment (start 161 66.2) (end 160.8 66) (width 2) (layer "F.Cu") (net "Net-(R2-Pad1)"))
 (segment (start 161 118) (end 161 66.2) (width 2) (layer "F.Cu") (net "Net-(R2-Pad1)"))
 (segment (start 186.2 66) (end 195.8 66) (width 2) (layer "F.Cu") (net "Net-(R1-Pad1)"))
 (segment (start 203.5 66) (end 200.17 62.67) (width 2) (layer "B.Cu") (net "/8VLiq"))
 (segment (start 175.99 58.69) (end 175.99 56.27) (width 2) (layer "B.Cu") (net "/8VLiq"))
 (segment (start 179.97 62.67) (end 175.99 58.69) (width 2) (layer "B.Cu") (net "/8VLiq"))
 (segment (start 221.2 66) (end 203.5 66) (width 2) (layer "B.Cu") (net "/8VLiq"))
 (segment (start 200.17 62.67) (end 179.97 62.67) (width 2) (layer "B.Cu") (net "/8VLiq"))
 (segment (start 226.5 69) (end 226.5 66.14) (width 2) (layer "B.Cu") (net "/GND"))
 (segment (start 226.5 66.14) (end 216.63 56.27) (width 2) (layer "B.Cu") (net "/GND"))
 (segment (start 210.5 126) (end 206 121.5) (width 2) (layer "B.Cu") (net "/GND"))
 (segment (start 206 89.5) (end 226.5 69) (width 2) (layer "B.Cu") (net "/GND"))
 (segment (start 221.09 126) (end 210.5 126) (width 2) (layer "B.Cu") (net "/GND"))
 (segment (start 206 121.5) (end 206 89.5) (width 2) (layer "B.Cu") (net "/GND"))
 (segment (start 226.55 120.54) (end 221.09 126) (width 2) (layer "B.Cu") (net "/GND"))
 (segment (start 229.3 82.35) (end 211.55 64.6) (width 2) (layer "F.Cu") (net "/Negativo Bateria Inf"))
 (segment (start 211.55 64.6) (end 211.55 56.27) (width 2) (layer "F.Cu") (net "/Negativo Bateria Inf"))
 (segment (start 229.3 82.35) (end 229.3 101.65) (width 2) (layer "F.Cu") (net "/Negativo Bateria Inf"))
 (segment (start 203.91 56.29) (end 203.93 56.27) (width 0.2) (layer "F.Cu") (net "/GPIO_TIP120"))
 (segment (start 222.46 115.46) (end 203.91 96.91) (width 0.2) (layer "F.Cu") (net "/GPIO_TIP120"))
 (segment (start 226.55 115.46) (end 222.46 115.46) (width 0.2) (layer "F.Cu") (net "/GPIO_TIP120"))
 (segment (start 203.91 96.91) (end 203.91 56.29) (width 0.2) (layer "F.Cu") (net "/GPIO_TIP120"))
 (segment (start 196.31 56.27) (end 196.31 56.558428) (width 2) (layer "F.Cu") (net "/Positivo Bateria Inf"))
 (segment (start 159 60.5) (end 156.4 63.1) (width 2) (layer "F.Cu") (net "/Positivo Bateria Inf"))
 (segment (start 156.4 63.1) (end 156.4 82.35) (width 2) (layer "F.Cu") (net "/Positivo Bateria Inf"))
 (segment (start 192.368428 60.5) (end 159 60.5) (width 2) (layer "F.Cu") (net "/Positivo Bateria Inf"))
 (segment (start 196.31 56.558428) (end 192.368428 60.5) (width 2) (layer "F.Cu") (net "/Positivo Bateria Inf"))
 (segment (start 156.4 101.65) (end 156.4 82.35) (width 2) (layer "B.Cu") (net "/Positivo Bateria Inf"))
 (segment (start 226.55 118) (end 220.2 118) (width 2) (layer "F.Cu") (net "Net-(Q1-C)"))
 (segment (start 194.8 118) (end 186.4 118) (width 2) (layer "F.Cu") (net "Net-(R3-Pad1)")))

